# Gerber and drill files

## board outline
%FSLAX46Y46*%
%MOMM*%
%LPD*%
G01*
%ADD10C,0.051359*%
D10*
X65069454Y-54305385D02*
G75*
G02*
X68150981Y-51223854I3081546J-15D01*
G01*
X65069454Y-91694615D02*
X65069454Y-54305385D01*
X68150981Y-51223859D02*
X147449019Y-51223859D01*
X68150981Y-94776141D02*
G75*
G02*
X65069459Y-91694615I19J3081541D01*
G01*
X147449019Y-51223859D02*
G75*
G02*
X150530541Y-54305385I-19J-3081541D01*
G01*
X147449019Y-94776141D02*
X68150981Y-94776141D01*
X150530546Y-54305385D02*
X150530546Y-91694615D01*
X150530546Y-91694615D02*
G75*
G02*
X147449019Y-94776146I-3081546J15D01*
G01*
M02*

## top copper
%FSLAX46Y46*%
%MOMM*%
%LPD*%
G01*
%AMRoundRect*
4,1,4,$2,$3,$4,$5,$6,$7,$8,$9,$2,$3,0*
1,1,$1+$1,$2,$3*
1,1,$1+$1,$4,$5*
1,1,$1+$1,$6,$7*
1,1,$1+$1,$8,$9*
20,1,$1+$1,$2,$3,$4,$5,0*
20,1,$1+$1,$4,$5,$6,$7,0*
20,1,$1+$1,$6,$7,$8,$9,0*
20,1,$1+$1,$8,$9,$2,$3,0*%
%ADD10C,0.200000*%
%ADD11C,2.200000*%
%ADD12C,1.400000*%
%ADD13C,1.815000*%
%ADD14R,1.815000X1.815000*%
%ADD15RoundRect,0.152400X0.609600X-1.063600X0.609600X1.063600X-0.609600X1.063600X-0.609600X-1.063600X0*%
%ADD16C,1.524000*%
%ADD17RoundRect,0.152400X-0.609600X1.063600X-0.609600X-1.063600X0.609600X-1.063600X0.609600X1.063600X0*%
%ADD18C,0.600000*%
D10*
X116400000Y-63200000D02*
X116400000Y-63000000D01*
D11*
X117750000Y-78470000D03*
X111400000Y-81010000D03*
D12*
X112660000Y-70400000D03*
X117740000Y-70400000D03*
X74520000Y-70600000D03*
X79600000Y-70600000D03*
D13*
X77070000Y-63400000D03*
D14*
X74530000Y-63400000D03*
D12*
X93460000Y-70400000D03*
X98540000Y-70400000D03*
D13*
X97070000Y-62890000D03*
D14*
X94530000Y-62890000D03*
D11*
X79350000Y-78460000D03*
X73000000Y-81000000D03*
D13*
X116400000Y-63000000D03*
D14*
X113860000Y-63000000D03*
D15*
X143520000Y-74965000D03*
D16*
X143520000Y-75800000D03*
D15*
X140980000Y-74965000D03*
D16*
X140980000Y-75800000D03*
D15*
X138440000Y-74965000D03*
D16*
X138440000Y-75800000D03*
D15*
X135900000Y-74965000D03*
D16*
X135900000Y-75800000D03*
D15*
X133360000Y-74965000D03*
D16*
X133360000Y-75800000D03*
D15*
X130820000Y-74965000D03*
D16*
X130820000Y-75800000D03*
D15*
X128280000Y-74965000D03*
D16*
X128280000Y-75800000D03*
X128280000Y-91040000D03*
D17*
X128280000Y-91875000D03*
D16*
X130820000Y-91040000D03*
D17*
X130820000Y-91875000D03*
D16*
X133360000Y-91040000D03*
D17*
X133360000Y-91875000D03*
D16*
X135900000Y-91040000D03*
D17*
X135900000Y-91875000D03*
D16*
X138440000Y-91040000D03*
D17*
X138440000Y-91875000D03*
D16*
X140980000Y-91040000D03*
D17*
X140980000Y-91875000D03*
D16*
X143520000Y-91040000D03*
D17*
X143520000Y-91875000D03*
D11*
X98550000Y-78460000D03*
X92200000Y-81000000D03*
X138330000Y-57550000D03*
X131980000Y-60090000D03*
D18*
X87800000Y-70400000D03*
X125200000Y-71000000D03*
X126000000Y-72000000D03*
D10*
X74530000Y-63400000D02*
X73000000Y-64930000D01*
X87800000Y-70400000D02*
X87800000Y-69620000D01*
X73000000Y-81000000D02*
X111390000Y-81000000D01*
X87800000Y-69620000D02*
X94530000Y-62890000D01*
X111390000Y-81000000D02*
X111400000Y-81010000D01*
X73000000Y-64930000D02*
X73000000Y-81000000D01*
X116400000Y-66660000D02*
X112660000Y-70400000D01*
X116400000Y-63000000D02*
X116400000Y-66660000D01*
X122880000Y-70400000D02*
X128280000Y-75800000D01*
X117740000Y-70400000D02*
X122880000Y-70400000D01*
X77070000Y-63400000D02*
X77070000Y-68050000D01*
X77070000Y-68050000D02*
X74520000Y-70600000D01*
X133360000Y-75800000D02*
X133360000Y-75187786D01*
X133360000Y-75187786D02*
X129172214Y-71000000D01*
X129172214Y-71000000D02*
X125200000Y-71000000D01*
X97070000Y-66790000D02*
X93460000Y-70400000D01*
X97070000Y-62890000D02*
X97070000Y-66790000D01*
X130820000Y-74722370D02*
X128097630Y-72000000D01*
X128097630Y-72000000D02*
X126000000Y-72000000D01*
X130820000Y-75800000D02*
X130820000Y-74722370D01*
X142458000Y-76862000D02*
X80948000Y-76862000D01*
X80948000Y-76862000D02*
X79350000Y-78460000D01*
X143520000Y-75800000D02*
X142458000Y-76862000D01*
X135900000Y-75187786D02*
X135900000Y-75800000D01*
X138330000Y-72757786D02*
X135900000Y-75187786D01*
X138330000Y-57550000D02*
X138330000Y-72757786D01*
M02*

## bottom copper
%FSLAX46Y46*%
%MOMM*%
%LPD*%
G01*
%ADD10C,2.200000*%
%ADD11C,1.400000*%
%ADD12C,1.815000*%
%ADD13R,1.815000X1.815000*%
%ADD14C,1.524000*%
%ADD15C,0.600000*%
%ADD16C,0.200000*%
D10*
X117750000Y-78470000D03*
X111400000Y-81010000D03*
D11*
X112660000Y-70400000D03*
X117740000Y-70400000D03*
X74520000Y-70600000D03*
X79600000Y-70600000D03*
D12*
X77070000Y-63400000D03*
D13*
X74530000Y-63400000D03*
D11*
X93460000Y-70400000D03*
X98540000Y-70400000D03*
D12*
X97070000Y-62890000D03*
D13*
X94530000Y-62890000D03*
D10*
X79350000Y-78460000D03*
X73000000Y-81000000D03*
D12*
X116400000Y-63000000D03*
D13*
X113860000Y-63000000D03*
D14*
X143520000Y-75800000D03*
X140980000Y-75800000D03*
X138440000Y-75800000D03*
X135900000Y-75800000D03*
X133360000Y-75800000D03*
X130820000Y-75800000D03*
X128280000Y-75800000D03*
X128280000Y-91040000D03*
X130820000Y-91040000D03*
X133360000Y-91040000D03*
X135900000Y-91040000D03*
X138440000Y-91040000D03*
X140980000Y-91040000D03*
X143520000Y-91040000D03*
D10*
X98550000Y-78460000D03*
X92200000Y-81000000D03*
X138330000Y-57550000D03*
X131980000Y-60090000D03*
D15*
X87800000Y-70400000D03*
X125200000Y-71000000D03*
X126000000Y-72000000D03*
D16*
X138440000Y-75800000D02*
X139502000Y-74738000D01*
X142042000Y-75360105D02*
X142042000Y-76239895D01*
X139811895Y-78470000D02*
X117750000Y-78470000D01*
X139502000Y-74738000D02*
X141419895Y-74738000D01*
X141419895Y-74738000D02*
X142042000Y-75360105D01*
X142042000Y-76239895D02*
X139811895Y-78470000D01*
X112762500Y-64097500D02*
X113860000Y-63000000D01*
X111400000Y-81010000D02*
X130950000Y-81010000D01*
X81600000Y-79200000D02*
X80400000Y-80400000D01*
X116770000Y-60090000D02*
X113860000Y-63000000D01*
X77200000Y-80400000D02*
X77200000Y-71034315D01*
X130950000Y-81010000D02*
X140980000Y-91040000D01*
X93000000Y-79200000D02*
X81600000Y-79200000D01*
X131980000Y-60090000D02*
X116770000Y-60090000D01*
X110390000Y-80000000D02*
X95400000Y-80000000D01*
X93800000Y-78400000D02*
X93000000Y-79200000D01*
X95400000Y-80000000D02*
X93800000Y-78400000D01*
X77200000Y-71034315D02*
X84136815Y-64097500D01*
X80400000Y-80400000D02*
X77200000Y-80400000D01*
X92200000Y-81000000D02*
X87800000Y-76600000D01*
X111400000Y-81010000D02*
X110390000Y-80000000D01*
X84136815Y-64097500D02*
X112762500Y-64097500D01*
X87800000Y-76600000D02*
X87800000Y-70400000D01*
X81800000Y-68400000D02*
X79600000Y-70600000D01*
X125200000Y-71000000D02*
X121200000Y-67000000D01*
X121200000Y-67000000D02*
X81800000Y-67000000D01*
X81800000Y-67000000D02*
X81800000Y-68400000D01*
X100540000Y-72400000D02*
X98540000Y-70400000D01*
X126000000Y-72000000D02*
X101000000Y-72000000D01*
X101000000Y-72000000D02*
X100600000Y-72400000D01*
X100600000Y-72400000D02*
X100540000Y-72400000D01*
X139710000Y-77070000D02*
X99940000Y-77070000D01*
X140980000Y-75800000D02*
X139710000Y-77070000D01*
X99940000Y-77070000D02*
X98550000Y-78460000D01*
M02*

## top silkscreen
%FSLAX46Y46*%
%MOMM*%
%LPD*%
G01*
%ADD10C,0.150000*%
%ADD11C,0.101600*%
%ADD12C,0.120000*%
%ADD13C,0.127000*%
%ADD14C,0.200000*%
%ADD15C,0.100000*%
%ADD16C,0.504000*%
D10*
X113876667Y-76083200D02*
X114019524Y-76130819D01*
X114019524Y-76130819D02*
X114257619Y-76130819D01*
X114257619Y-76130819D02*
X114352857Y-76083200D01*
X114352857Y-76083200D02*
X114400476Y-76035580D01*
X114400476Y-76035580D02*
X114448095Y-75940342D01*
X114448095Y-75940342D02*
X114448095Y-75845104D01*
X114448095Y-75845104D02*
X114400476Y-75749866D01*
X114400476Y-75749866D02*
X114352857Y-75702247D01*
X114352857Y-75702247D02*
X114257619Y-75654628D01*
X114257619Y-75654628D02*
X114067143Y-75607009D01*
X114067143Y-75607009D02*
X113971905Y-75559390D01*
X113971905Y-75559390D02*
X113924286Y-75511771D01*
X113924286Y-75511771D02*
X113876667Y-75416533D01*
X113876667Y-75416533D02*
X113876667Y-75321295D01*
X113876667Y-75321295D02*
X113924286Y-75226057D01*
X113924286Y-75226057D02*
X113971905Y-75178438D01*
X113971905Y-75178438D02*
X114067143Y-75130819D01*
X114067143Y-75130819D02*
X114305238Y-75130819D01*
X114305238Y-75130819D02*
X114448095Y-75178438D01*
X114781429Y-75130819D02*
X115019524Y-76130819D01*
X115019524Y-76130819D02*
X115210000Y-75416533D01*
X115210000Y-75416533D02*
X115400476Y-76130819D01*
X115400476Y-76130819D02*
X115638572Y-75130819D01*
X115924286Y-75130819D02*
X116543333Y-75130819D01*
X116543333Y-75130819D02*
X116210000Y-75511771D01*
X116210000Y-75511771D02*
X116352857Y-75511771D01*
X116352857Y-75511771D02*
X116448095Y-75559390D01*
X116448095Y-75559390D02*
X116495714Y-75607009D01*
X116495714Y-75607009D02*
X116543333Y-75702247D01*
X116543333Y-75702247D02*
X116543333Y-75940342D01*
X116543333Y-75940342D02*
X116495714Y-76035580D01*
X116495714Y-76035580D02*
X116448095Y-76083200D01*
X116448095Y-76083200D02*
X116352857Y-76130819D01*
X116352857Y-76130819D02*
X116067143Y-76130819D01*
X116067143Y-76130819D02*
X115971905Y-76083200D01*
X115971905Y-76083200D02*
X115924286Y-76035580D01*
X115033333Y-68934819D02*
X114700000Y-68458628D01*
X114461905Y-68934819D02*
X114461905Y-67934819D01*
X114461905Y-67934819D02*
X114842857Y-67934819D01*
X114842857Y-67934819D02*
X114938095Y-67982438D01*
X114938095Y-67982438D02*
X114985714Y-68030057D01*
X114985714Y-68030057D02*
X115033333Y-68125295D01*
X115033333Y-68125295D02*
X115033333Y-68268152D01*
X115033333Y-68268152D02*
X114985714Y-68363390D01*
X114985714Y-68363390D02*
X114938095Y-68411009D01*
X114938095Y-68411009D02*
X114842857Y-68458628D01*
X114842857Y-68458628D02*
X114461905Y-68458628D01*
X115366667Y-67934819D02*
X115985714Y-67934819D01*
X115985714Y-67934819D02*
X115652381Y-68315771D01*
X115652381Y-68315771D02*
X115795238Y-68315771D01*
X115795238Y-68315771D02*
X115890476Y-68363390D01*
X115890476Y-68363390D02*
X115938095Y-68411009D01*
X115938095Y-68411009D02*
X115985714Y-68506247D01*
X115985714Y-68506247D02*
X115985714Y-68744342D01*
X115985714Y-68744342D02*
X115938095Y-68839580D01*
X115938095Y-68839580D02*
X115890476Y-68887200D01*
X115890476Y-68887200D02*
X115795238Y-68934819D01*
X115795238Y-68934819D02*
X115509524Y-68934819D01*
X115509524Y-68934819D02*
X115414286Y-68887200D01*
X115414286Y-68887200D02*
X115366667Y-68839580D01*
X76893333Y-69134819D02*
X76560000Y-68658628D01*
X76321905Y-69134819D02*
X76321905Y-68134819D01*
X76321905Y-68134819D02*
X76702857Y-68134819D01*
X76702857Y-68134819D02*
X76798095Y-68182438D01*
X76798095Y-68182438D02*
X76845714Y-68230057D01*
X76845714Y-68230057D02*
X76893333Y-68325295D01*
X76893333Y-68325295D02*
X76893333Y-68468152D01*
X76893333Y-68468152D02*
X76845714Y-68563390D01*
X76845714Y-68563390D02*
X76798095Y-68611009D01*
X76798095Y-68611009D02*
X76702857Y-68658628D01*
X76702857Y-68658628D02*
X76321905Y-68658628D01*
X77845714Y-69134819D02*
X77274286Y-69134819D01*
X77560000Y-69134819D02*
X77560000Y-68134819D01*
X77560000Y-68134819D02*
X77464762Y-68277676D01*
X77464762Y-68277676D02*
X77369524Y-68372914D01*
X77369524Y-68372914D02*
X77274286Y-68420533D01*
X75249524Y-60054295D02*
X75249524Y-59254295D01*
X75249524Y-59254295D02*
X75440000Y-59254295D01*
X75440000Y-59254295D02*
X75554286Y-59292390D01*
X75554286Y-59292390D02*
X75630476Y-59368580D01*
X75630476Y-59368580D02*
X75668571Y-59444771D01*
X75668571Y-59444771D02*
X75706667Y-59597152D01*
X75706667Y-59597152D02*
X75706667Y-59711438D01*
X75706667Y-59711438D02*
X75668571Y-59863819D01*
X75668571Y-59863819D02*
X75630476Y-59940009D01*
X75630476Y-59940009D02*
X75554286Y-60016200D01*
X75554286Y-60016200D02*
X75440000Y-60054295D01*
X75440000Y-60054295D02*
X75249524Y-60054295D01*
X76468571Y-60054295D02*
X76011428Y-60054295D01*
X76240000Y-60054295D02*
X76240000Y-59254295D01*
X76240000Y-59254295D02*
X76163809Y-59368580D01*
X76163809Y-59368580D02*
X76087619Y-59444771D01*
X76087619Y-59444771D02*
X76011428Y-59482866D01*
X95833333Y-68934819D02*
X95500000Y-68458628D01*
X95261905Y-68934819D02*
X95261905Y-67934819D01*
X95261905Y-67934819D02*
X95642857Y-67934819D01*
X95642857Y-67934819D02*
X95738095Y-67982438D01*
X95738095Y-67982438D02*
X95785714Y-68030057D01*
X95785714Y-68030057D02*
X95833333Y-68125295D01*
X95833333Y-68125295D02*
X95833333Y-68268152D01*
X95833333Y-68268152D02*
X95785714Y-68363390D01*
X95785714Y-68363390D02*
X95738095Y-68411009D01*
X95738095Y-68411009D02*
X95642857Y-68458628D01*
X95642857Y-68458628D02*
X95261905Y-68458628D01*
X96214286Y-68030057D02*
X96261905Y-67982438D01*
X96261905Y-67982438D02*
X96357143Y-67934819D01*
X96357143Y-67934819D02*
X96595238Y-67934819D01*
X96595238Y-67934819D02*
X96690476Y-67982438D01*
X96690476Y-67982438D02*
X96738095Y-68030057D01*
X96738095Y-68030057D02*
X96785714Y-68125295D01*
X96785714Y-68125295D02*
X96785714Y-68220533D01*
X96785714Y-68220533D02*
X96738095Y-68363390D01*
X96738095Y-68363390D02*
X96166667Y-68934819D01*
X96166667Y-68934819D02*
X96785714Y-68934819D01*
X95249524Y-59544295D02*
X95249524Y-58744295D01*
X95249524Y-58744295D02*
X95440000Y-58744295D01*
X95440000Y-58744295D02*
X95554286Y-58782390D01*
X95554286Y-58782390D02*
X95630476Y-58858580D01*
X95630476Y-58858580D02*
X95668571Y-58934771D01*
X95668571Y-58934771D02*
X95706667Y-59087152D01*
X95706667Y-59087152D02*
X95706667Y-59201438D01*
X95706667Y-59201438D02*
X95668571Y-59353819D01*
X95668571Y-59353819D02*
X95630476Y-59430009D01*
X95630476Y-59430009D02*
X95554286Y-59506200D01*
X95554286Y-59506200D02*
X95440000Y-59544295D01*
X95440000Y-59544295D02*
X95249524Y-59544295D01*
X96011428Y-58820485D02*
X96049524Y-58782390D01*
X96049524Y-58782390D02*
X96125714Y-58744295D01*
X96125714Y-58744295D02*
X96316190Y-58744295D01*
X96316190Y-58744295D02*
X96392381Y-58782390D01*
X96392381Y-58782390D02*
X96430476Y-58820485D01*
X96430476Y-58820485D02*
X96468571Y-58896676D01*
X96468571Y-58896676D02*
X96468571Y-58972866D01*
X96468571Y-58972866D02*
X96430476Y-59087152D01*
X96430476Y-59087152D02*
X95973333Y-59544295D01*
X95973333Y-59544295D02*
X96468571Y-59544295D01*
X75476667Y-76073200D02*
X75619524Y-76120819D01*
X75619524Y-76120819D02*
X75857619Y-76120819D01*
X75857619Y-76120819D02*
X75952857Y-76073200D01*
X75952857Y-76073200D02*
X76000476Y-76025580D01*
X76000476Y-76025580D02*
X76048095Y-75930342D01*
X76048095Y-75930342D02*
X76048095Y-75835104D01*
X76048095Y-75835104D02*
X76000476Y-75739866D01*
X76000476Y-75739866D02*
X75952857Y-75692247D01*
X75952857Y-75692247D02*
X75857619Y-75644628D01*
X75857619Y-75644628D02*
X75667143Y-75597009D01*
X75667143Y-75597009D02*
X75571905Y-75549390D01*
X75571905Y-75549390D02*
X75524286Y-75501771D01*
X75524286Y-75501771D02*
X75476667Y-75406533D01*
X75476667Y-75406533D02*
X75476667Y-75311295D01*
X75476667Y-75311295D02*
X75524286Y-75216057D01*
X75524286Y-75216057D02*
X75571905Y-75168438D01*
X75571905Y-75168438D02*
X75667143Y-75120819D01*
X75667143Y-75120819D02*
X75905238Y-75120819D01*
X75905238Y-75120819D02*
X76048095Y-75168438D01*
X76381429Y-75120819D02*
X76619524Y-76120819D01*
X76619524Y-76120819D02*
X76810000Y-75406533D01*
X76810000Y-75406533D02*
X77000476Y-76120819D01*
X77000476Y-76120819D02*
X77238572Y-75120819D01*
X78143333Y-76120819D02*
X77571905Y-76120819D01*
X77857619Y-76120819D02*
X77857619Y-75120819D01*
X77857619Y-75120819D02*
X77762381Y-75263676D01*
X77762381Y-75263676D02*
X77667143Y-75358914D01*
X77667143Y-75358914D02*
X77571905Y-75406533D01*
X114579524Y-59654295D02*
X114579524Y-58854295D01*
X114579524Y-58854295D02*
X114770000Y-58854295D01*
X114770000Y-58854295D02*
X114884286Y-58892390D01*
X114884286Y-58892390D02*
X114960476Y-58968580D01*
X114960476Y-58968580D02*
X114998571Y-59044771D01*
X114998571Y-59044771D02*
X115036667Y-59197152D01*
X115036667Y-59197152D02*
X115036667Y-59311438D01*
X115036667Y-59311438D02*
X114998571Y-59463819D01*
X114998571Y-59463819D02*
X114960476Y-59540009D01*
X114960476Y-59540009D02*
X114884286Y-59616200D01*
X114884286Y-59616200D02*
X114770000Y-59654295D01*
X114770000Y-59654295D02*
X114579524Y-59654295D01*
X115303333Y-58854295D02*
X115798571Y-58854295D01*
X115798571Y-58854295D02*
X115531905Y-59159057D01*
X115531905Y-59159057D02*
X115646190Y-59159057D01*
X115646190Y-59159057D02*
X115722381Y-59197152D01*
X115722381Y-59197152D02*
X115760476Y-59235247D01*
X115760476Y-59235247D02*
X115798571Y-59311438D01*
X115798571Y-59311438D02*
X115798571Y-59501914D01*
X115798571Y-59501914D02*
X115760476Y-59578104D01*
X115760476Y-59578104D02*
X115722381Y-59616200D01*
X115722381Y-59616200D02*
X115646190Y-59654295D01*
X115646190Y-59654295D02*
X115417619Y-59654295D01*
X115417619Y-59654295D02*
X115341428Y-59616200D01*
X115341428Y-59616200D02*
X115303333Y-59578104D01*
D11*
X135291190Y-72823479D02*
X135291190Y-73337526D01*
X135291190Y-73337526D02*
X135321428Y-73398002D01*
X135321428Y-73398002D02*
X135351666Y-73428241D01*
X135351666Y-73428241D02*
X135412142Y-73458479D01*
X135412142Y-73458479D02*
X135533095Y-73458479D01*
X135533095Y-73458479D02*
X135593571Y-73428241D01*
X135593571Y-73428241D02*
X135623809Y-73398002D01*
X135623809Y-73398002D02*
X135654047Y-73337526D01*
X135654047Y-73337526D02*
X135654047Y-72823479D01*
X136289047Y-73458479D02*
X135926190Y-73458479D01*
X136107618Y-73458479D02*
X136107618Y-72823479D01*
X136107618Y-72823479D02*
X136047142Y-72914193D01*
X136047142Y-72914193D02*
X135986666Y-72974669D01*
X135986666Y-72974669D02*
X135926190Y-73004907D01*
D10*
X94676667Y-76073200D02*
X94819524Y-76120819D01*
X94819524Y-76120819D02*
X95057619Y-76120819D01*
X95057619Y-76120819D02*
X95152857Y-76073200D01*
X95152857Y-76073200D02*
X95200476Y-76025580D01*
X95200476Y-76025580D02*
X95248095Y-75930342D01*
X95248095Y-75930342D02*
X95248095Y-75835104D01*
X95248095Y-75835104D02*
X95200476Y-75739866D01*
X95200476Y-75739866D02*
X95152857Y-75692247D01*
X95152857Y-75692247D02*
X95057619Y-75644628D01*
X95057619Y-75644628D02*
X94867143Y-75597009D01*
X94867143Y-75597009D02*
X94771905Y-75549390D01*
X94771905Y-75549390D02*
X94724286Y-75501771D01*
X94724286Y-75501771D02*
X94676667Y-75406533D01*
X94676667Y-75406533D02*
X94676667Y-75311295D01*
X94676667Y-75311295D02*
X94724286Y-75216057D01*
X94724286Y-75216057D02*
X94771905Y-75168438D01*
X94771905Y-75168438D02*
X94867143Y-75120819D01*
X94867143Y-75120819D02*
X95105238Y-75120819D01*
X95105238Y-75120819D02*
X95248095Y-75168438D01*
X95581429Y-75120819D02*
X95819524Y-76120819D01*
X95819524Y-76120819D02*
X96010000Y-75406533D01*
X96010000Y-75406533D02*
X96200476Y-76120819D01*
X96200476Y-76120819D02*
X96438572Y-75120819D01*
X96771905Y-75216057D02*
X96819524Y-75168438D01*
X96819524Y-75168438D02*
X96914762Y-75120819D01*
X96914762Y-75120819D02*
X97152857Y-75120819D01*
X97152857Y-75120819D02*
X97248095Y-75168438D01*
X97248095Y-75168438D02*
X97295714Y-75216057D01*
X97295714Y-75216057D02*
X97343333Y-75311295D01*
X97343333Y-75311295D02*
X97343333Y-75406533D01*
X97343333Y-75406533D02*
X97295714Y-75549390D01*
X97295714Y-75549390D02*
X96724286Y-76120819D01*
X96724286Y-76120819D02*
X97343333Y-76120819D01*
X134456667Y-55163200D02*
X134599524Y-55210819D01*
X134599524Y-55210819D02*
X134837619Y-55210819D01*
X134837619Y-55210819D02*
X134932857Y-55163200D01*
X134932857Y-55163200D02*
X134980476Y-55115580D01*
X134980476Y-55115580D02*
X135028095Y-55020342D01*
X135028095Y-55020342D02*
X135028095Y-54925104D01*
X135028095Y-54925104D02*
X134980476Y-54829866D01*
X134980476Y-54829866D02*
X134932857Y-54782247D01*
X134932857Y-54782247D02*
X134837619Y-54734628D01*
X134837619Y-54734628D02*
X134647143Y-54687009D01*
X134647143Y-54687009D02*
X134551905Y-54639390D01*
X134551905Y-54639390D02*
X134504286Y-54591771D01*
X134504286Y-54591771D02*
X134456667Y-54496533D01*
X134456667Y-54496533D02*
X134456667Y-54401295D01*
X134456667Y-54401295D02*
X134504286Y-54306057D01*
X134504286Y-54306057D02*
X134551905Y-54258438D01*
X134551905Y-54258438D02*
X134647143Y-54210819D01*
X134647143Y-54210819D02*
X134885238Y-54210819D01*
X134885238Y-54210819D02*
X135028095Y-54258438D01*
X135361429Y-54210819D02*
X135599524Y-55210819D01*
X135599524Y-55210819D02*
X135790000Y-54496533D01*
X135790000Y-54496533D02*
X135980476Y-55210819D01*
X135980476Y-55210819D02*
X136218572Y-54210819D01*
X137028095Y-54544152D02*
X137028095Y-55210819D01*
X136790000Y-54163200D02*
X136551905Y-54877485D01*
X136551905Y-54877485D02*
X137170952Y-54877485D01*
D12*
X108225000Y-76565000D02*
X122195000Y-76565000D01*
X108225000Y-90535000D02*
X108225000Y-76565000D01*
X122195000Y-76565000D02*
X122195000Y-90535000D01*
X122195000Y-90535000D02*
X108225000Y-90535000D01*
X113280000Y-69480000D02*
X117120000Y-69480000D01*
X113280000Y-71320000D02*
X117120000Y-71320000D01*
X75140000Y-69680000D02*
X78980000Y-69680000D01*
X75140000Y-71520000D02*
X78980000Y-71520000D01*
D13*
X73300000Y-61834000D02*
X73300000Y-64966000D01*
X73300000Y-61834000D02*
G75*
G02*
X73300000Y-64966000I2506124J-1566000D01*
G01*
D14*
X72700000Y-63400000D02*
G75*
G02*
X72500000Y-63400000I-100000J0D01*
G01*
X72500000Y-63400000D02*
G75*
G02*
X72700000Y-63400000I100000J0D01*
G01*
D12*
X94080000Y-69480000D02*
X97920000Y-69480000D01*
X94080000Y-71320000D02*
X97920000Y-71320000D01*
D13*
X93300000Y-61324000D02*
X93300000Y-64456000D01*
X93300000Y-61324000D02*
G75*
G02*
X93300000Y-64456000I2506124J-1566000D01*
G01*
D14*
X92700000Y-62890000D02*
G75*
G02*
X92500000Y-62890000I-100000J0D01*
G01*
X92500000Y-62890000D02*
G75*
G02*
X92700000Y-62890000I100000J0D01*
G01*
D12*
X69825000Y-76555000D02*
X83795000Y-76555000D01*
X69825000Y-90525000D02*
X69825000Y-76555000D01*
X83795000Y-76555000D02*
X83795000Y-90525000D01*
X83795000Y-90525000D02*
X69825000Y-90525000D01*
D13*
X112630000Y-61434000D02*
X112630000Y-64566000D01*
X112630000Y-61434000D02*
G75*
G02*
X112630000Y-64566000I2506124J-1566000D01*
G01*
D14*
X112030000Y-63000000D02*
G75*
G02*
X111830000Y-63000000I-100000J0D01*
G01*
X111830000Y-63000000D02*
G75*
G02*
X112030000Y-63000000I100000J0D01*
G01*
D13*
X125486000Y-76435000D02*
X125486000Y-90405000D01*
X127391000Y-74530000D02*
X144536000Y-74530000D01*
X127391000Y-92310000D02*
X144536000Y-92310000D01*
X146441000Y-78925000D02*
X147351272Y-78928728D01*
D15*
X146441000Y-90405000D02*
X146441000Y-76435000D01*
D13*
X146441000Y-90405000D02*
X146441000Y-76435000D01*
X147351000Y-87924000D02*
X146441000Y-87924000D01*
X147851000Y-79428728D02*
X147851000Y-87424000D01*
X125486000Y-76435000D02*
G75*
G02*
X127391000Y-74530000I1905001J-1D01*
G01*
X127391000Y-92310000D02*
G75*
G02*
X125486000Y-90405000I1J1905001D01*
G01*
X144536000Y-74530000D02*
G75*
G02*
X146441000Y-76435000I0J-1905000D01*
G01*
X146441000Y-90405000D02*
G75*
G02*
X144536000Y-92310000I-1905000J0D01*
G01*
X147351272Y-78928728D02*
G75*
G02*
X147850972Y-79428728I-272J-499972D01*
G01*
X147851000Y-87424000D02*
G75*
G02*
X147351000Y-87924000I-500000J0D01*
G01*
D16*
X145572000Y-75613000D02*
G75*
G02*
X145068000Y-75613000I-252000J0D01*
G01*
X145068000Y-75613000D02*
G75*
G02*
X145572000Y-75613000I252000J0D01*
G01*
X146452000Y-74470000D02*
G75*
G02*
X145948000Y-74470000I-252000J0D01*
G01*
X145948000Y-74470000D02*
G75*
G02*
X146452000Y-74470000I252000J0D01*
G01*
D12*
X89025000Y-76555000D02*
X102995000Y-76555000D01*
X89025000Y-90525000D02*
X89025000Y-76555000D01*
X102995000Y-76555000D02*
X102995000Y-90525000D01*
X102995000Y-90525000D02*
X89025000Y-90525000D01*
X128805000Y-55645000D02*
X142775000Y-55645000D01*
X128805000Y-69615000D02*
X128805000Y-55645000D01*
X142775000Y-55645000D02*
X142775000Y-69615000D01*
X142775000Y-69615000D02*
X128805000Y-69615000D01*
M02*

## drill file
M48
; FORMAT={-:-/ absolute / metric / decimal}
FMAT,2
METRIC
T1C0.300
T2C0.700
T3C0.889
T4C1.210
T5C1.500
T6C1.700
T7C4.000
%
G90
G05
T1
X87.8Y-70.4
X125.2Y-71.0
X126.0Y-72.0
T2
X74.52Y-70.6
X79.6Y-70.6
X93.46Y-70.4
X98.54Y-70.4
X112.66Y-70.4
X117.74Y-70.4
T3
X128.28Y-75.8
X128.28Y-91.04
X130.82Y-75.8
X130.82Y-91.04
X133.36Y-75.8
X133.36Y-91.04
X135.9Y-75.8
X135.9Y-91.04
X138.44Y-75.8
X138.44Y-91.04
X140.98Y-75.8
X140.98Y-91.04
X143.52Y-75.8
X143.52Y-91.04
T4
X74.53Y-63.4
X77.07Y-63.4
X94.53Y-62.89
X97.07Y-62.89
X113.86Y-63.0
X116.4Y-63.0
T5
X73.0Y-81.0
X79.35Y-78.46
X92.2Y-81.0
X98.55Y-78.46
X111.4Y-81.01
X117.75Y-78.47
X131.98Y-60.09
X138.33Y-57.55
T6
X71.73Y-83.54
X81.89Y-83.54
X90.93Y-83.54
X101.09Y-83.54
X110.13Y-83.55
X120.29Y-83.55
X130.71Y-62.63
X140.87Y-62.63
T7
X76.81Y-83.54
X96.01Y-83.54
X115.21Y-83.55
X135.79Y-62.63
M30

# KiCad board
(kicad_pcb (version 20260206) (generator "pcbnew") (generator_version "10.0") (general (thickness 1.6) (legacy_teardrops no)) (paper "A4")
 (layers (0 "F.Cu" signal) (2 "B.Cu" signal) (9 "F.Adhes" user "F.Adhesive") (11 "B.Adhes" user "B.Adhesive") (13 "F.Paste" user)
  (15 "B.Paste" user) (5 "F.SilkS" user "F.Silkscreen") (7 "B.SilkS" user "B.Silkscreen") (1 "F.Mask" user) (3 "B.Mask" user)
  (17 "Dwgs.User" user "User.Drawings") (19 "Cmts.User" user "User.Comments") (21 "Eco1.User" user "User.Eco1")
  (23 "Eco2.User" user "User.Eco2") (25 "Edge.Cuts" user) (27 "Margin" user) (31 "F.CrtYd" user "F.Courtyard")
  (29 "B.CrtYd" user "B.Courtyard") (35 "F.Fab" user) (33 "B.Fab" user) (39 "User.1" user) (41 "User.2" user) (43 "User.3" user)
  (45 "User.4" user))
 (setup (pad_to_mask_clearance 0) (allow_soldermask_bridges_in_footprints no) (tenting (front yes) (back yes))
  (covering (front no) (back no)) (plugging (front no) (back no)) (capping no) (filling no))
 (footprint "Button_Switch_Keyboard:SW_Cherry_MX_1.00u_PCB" (layer "F.Cu") (at 117.75 78.47)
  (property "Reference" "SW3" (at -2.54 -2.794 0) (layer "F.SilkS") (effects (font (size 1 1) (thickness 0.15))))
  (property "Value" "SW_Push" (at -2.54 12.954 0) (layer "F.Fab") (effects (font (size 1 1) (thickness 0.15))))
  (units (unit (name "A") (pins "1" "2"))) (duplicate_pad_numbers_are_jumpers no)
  (fp_line (start -9.525 -1.905) (end 4.445 -1.905) (stroke (width 0.12) (type solid)) (layer "F.SilkS"))
  (fp_line (start -9.525 12.065) (end -9.525 -1.905) (stroke (width 0.12) (type solid)) (layer "F.SilkS"))
  (fp_line (start 4.445 -1.905) (end 4.445 12.065) (stroke (width 0.12) (type solid)) (layer "F.SilkS"))
  (fp_line (start 4.445 12.065) (end -9.525 12.065) (stroke (width 0.12) (type solid)) (layer "F.SilkS"))
  (pad "" np_thru_hole circle (at -7.62 5.08) (size 1.7 1.7) (drill 1.7) (layers "*.Cu" "*.Mask"))
  (pad "" np_thru_hole circle (at -2.54 5.08) (size 4 4) (drill 4) (layers "*.Cu" "*.Mask"))
  (pad "" np_thru_hole circle (at 2.54 5.08) (size 1.7 1.7) (drill 1.7) (layers "*.Cu" "*.Mask"))
  (pad "1" thru_hole circle (at 0 0) (size 2.2 2.2) (drill 1.5) (layers "*.Cu" "*.Mask") (remove_unused_layers no)
   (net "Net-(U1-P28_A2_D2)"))
  (pad "2" thru_hole circle (at -6.35 2.54) (size 2.2 2.2) (drill 1.5) (layers "*.Cu" "*.Mask") (remove_unused_layers no) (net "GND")))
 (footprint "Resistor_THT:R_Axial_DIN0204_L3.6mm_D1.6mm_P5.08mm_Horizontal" (layer "F.Cu") (at 112.66 70.4)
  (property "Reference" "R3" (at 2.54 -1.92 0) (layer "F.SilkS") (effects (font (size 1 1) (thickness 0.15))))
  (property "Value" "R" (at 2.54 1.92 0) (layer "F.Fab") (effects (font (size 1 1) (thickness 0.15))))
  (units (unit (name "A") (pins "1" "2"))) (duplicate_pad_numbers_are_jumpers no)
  (fp_line (start 0.62 -0.92) (end 4.46 -0.92) (stroke (width 0.12) (type solid)) (layer "F.SilkS"))
  (fp_line (start 0.62 0.92) (end 4.46 0.92) (stroke (width 0.12) (type solid)) (layer "F.SilkS"))
  (pad "1" thru_hole circle (at 0 0) (size 1.4 1.4) (drill 0.7) (layers "*.Cu" "*.Mask") (remove_unused_layers no) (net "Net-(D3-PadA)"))
  (pad "2" thru_hole circle (at 5.08 0) (size 1.4 1.4) (drill 0.7) (layers "*.Cu" "*.Mask") (remove_unused_layers no)
   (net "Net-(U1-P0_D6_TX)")))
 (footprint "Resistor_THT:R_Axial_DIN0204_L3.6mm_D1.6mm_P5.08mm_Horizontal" (layer "F.Cu") (at 74.52 70.6)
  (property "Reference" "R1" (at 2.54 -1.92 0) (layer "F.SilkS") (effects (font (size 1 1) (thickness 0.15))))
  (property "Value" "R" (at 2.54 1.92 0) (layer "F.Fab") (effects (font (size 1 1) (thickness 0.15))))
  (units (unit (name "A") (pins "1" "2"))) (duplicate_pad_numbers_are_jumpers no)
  (fp_line (start 0.62 -0.92) (end 4.46 -0.92) (stroke (width 0.12) (type solid)) (layer "F.SilkS"))
  (fp_line (start 0.62 0.92) (end 4.46 0.92) (stroke (width 0.12) (type solid)) (layer "F.SilkS"))
  (pad "1" thru_hole circle (at 0 0) (size 1.4 1.4) (drill 0.7) (layers "*.Cu" "*.Mask") (remove_unused_layers no) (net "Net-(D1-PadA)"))
  (pad "2" thru_hole circle (at 5.08 0) (size 1.4 1.4) (drill 0.7) (layers "*.Cu" "*.Mask") (remove_unused_layers no)
   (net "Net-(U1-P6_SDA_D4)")))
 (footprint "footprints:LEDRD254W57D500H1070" (layer "F.Cu") (at 75.8 63.4)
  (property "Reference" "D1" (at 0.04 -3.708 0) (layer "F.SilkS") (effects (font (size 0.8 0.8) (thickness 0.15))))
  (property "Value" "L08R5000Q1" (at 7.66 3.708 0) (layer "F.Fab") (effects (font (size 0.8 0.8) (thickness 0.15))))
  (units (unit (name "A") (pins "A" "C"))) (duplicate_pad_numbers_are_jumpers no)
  (fp_line (start -2.5 -1.566) (end -2.5 1.566) (stroke (width 0.127) (type solid)) (layer "F.SilkS"))
  (fp_arc (start -2.5 -1.566) (mid 2.961291 0) (end -2.5 1.566) (stroke (width 0.127) (type solid)) (layer "F.SilkS"))
  (fp_circle (center -3.2 0) (end -3.1 0) (stroke (width 0.2) (type solid)) (fill no) (layer "F.SilkS"))
  (pad "A" thru_hole circle (at 1.27 0) (size 1.815 1.815) (drill 1.21) (layers "*.Cu" "*.Mask") (remove_unused_layers no)
   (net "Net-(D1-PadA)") (solder_mask_margin 0.102))
  (pad "C" thru_hole rect (at -1.27 0) (size 1.815 1.815) (drill 1.21) (layers "*.Cu" "*.Mask") (remove_unused_layers no) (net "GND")
   (solder_mask_margin 0.102)))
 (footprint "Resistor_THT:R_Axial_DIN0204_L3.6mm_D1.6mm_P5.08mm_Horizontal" (layer "F.Cu") (at 93.46 70.4)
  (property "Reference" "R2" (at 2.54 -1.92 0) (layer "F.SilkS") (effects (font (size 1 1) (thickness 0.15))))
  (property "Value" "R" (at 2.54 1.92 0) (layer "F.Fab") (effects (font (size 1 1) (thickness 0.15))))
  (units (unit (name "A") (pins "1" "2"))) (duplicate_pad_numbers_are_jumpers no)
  (fp_line (start 0.62 -0.92) (end 4.46 -0.92) (stroke (width 0.12) (type solid)) (layer "F.SilkS"))
  (fp_line (start 0.62 0.92) (end 4.46 0.92) (stroke (width 0.12) (type solid)) (layer "F.SilkS"))
  (pad "1" thru_hole circle (at 0 0) (size 1.4 1.4) (drill 0.7) (layers "*.Cu" "*.Mask") (remove_unused_layers no) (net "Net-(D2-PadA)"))
  (pad "2" thru_hole circle (at 5.08 0) (size 1.4 1.4) (drill 0.7) (layers "*.Cu" "*.Mask") (remove_unused_layers no)
   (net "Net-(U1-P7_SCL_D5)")))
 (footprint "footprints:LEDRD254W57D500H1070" (layer "F.Cu") (at 95.8 62.89)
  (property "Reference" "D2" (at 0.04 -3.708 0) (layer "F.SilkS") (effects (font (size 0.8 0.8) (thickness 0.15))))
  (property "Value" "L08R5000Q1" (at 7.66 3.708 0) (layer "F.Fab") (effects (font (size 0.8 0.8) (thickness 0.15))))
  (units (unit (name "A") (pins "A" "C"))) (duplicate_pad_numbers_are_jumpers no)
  (fp_line (start -2.5 -1.566) (end -2.5 1.566) (stroke (width 0.127) (type solid)) (layer "F.SilkS"))
  (fp_arc (start -2.5 -1.566) (mid 2.961291 0) (end -2.5 1.566) (stroke (width 0.127) (type solid)) (layer "F.SilkS"))
  (fp_circle (center -3.2 0) (end -3.1 0) (stroke (width 0.2) (type solid)) (fill no) (layer "F.SilkS"))
  (pad "A" thru_hole circle (at 1.27 0) (size 1.815 1.815) (drill 1.21) (layers "*.Cu" "*.Mask") (remove_unused_layers no)
   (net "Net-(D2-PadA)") (solder_mask_margin 0.102))
  (pad "C" thru_hole rect (at -1.27 0) (size 1.815 1.815) (drill 1.21) (layers "*.Cu" "*.Mask") (remove_unused_layers no) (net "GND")
   (solder_mask_margin 0.102)))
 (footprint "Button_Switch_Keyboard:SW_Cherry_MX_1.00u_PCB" (layer "F.Cu") (at 79.35 78.46)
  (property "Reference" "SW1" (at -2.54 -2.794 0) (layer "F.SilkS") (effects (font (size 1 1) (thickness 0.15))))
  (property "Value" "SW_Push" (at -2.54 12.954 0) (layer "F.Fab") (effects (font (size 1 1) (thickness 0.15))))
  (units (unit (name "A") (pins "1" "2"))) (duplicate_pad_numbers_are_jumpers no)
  (fp_line (start -9.525 -1.905) (end 4.445 -1.905) (stroke (width 0.12) (type solid)) (layer "F.SilkS"))
  (fp_line (start -9.525 12.065) (end -9.525 -1.905) (stroke (width 0.12) (type solid)) (layer "F.SilkS"))
  (fp_line (start 4.445 -1.905) (end 4.445 12.065) (stroke (width 0.12) (type solid)) (layer "F.SilkS"))
  (fp_line (start 4.445 12.065) (end -9.525 12.065) (stroke (width 0.12) (type solid)) (layer "F.SilkS"))
  (pad "" np_thru_hole circle (at -7.62 5.08) (size 1.7 1.7) (drill 1.7) (layers "*.Cu" "*.Mask"))
  (pad "" np_thru_hole circle (at -2.54 5.08) (size 4 4) (drill 4) (layers "*.Cu" "*.Mask"))
  (pad "" np_thru_hole circle (at 2.54 5.08) (size 1.7 1.7) (drill 1.7) (layers "*.Cu" "*.Mask"))
  (pad "1" thru_hole circle (at 0 0) (size 2.2 2.2) (drill 1.5) (layers "*.Cu" "*.Mask") (remove_unused_layers no)
   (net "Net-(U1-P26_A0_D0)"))
  (pad "2" thru_hole circle (at -6.35 2.54) (size 2.2 2.2) (drill 1.5) (layers "*.Cu" "*.Mask") (remove_unused_layers no) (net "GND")))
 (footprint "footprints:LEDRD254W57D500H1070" (layer "F.Cu") (at 115.13 63)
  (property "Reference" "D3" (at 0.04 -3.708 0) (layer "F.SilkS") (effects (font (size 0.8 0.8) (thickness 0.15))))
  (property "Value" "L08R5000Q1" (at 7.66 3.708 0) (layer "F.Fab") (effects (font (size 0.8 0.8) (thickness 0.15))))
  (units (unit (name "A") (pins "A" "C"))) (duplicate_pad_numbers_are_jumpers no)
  (fp_line (start -2.5 -1.566) (end -2.5 1.566) (stroke (width 0.127) (type solid)) (layer "F.SilkS"))
  (fp_arc (start -2.5 -1.566) (mid 2.961291 0) (end -2.5 1.566) (stroke (width 0.127) (type solid)) (layer "F.SilkS"))
  (fp_circle (center -3.2 0) (end -3.1 0) (stroke (width 0.2) (type solid)) (fill no) (layer "F.SilkS"))
  (pad "A" thru_hole circle (at 1.27 0) (size 1.815 1.815) (drill 1.21) (layers "*.Cu" "*.Mask") (remove_unused_layers no)
   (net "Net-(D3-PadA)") (solder_mask_margin 0.102))
  (pad "C" thru_hole rect (at -1.27 0) (size 1.815 1.815) (drill 1.21) (layers "*.Cu" "*.Mask") (remove_unused_layers no) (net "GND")
   (solder_mask_margin 0.102)))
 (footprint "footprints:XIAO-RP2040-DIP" (layer "F.Cu") (at 135.9 83.42)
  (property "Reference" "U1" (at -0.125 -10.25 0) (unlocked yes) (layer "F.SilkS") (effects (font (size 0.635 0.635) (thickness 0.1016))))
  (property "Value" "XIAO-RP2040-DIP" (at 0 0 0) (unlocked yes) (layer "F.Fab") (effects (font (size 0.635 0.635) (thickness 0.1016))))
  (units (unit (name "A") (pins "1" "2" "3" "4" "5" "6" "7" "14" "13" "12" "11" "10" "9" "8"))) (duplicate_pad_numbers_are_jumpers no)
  (fp_line (start -10.414 -6.985) (end -10.414 6.985) (stroke (width 0.127) (type solid)) (layer "F.SilkS"))
  (fp_line (start -8.509 -8.89) (end 8.636 -8.89) (stroke (width 0.127) (type solid)) (layer "F.SilkS"))
  (fp_line (start -8.509 8.89) (end 8.636 8.89) (stroke (width 0.127) (type solid)) (layer "F.SilkS"))
  (fp_line (start 10.541 -4.495) (end 11.451272 -4.491272) (stroke (width 0.127) (type solid)) (layer "F.SilkS"))
  (fp_line (start 10.541 6.985) (end 10.541 -6.985) (stroke (width 0.1) (type solid)) (layer "F.SilkS"))
  (fp_line (start 10.541 6.985) (end 10.541 -6.985) (stroke (width 0.127) (type solid)) (layer "F.SilkS"))
  (fp_line (start 11.451 4.504) (end 10.541 4.504) (stroke (width 0.127) (type solid)) (layer "F.SilkS"))
  (fp_line (start 11.951 -3.991272) (end 11.951 4.004) (stroke (width 0.127) (type solid)) (layer "F.SilkS"))
  (fp_arc (start -10.414 -6.985) (mid -9.856038 -8.332038) (end -8.509 -8.89) (stroke (width 0.127) (type solid)) (layer "F.SilkS"))
  (fp_arc (start -8.509 8.89) (mid -9.856038 8.332038) (end -10.414 6.985) (stroke (width 0.127) (type solid)) (layer "F.SilkS"))
  (fp_arc (start 8.636 -8.89) (mid 9.983038 -8.332038) (end 10.541 -6.985) (stroke (width 0.127) (type solid)) (layer "F.SilkS"))
  (fp_arc (start 10.541 6.985) (mid 9.983038 8.332038) (end 8.636 8.89) (stroke (width 0.127) (type solid)) (layer "F.SilkS"))
  (fp_arc (start 11.451272 -4.491272) (mid 11.804644 -4.344724) (end 11.951 -3.991272) (stroke (width 0.127) (type default))
   (layer "F.SilkS"))
  (fp_arc (start 11.951 4.004) (mid 11.804553 4.357553) (end 11.451 4.504) (stroke (width 0.127) (type default)) (layer "F.SilkS"))
  (fp_circle (center 9.42 -7.807) (end 9.674 -7.807) (stroke (width 0.5) (type solid)) (fill yes) (layer "F.SilkS"))
  (fp_circle (center 10.3 -8.95) (end 10.554 -8.95) (stroke (width 0.5) (type solid)) (fill yes) (layer "F.SilkS"))
  (pad "1" smd roundrect (at 7.62 -8.455 90) (size 2.432 1.524) (layers "F.Cu" "F.Mask") (roundrect_rratio 0.1) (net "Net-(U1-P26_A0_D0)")
   (thermal_bridge_angle 45))
  (pad "1" thru_hole circle (at 7.62 -7.62 90) (size 1.524 1.524) (drill 0.889) (layers "*.Cu" "*.Mask") (remove_unused_layers no)
   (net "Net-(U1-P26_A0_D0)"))
  (pad "2" smd roundrect (at 5.08 -8.455 90) (size 2.432 1.524) (layers "F.Cu" "F.Mask") (roundrect_rratio 0.1) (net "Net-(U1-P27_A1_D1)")
   (thermal_bridge_angle 45))
  (pad "2" thru_hole circle (at 5.08 -7.62 90) (size 1.524 1.524) (drill 0.889) (layers "*.Cu" "*.Mask") (remove_unused_layers no)
   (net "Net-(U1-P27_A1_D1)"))
  (pad "3" smd roundrect (at 2.54 -8.455 90) (size 2.432 1.524) (layers "F.Cu" "F.Mask") (roundrect_rratio 0.1) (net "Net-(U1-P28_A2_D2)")
   (thermal_bridge_angle 45))
  (pad "3" thru_hole circle (at 2.54 -7.62 90) (size 1.524 1.524) (drill 0.889) (layers "*.Cu" "*.Mask") (remove_unused_layers no)
   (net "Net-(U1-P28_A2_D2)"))
  (pad "4" smd roundrect (at 0 -8.455 90) (size 2.432 1.524) (layers "F.Cu" "F.Mask") (roundrect_rratio 0.1) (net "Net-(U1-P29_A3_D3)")
   (thermal_bridge_angle 45))
  (pad "4" thru_hole circle (at 0 -7.62 90) (size 1.524 1.524) (drill 0.889) (layers "*.Cu" "*.Mask") (remove_unused_layers no)
   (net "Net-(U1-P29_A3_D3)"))
  (pad "5" smd roundrect (at -2.54 -8.455 90) (size 2.432 1.524) (layers "F.Cu" "F.Mask") (roundrect_rratio 0.1) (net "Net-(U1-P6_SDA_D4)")
   (thermal_bridge_angle 45))
  (pad "5" thru_hole circle (at -2.54 -7.62 90) (size 1.524 1.524) (drill 0.889) (layers "*.Cu" "*.Mask") (remove_unused_layers no)
   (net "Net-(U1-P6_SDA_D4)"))
  (pad "6" smd roundrect (at -5.08 -8.455 90) (size 2.432 1.524) (layers "F.Cu" "F.Mask") (roundrect_rratio 0.1) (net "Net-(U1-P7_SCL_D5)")
   (thermal_bridge_angle 45))
  (pad "6" thru_hole circle (at -5.08 -7.62 90) (size 1.524 1.524) (drill 0.889) (layers "*.Cu" "*.Mask") (remove_unused_layers no)
   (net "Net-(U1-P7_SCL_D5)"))
  (pad "7" smd roundrect (at -7.62 -8.455 90) (size 2.432 1.524) (layers "F.Cu" "F.Mask") (roundrect_rratio 0.1) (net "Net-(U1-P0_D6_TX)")
   (thermal_bridge_angle 45))
  (pad "7" thru_hole circle (at -7.62 -7.62 90) (size 1.524 1.524) (drill 0.889) (layers "*.Cu" "*.Mask") (remove_unused_layers no)
   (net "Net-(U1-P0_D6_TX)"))
  (pad "8" thru_hole circle (at -7.62 7.62 270) (size 1.524 1.524) (drill 0.889) (layers "*.Cu" "*.Mask") (remove_unused_layers no)
   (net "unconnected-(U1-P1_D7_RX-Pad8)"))
  (pad "8" smd roundrect (at -7.62 8.455 270) (size 2.432 1.524) (layers "F.Cu" "F.Mask") (roundrect_rratio 0.1)
   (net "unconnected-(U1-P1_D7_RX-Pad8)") (thermal_bridge_angle 45))
  (pad "9" thru_hole circle (at -5.08 7.62 270) (size 1.524 1.524) (drill 0.889) (layers "*.Cu" "*.Mask") (remove_unused_layers no)
   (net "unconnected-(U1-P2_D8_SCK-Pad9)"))
  (pad "9" smd roundrect (at -5.08 8.455 270) (size 2.432 1.524) (layers "F.Cu" "F.Mask") (roundrect_rratio 0.1)
   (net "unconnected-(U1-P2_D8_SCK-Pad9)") (thermal_bridge_angle 45))
  (pad "10" thru_hole circle (at -2.54 7.62 270) (size 1.524 1.524) (drill 0.889) (layers "*.Cu" "*.Mask") (remove_unused_layers no)
   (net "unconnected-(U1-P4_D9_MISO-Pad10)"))
  (pad "10" smd roundrect (at -2.54 8.455 270) (size 2.432 1.524) (layers "F.Cu" "F.Mask") (roundrect_rratio 0.1)
   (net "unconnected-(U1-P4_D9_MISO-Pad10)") (thermal_bridge_angle 45))
  (pad "11" thru_hole circle (at 0 7.62 270) (size 1.524 1.524) (drill 0.889) (layers "*.Cu" "*.Mask") (remove_unused_layers no)
   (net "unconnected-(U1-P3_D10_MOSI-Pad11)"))
  (pad "11" smd roundrect (at 0 8.455 270) (size 2.432 1.524) (layers "F.Cu" "F.Mask") (roundrect_rratio 0.1)
   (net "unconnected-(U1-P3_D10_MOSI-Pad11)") (thermal_bridge_angle 45))
  (pad "12" thru_hole circle (at 2.54 7.62 270) (size 1.524 1.524) (drill 0.889) (layers "*.Cu" "*.Mask") (remove_unused_layers no)
   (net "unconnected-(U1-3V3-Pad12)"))
  (pad "12" smd roundrect (at 2.54 8.455 270) (size 2.432 1.524) (layers "F.Cu" "F.Mask") (roundrect_rratio 0.1)
   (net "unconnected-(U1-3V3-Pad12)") (thermal_bridge_angle 45))
  (pad "13" thru_hole circle (at 5.08 7.62 270) (size 1.524 1.524) (drill 0.889) (layers "*.Cu" "*.Mask") (remove_unused_layers no)
   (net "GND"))
  (pad "13" smd roundrect (at 5.08 8.455 270) (size 2.432 1.524) (layers "F.Cu" "F.Mask") (roundrect_rratio 0.1) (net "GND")
   (thermal_bridge_angle 45))
  (pad "14" thru_hole circle (at 7.62 7.62 270) (size 1.524 1.524) (drill 0.889) (layers "*.Cu" "*.Mask") (remove_unused_layers no)
   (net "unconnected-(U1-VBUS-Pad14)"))
  (pad "14" smd roundrect (at 7.62 8.455 270) (size 2.432 1.524) (layers "F.Cu" "F.Mask") (roundrect_rratio 0.1)
   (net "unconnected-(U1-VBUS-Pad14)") (thermal_bridge_angle 45)))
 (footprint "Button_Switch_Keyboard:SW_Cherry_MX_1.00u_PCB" (layer "F.Cu") (at 98.55 78.46)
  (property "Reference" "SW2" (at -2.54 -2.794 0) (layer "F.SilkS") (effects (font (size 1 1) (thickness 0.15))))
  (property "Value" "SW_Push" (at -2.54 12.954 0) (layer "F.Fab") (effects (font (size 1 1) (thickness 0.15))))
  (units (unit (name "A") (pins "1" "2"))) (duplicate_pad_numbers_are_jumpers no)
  (fp_line (start -9.525 -1.905) (end 4.445 -1.905) (stroke (width 0.12) (type solid)) (layer "F.SilkS"))
  (fp_line (start -9.525 12.065) (end -9.525 -1.905) (stroke (width 0.12) (type solid)) (layer "F.SilkS"))
  (fp_line (start 4.445 -1.905) (end 4.445 12.065) (stroke (width 0.12) (type solid)) (layer "F.SilkS"))
  (fp_line (start 4.445 12.065) (end -9.525 12.065) (stroke (width 0.12) (type solid)) (layer "F.SilkS"))
  (pad "" np_thru_hole circle (at -7.62 5.08) (size 1.7 1.7) (drill 1.7) (layers "*.Cu" "*.Mask"))
  (pad "" np_thru_hole circle (at -2.54 5.08) (size 4 4) (drill 4) (layers "*.Cu" "*.Mask"))
  (pad "" np_thru_hole circle (at 2.54 5.08) (size 1.7 1.7) (drill 1.7) (layers "*.Cu" "*.Mask"))
  (pad "1" thru_hole circle (at 0 0) (size 2.2 2.2) (drill 1.5) (layers "*.Cu" "*.Mask") (remove_unused_layers no)
   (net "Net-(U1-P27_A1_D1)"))
  (pad "2" thru_hole circle (at -6.35 2.54) (size 2.2 2.2) (drill 1.5) (layers "*.Cu" "*.Mask") (remove_unused_layers no) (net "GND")))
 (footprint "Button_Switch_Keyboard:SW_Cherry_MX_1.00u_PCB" (layer "F.Cu") (at 138.33 57.55)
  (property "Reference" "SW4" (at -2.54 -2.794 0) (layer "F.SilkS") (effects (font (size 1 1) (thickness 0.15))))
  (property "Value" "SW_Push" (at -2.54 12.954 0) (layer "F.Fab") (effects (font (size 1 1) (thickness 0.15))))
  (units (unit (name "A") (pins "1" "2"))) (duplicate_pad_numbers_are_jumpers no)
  (fp_line (start -9.525 -1.905) (end 4.445 -1.905) (stroke (width 0.12) (type solid)) (layer "F.SilkS"))
  (fp_line (start -9.525 12.065) (end -9.525 -1.905) (stroke (width 0.12) (type solid)) (layer "F.SilkS"))
  (fp_line (start 4.445 -1.905) (end 4.445 12.065) (stroke (width 0.12) (type solid)) (layer "F.SilkS"))
  (fp_line (start 4.445 12.065) (end -9.525 12.065) (stroke (width 0.12) (type solid)) (layer "F.SilkS"))
  (pad "" np_thru_hole circle (at -7.62 5.08) (size 1.7 1.7) (drill 1.7) (layers "*.Cu" "*.Mask"))
  (pad "" np_thru_hole circle (at -2.54 5.08) (size 4 4) (drill 4) (layers "*.Cu" "*.Mask"))
  (pad "" np_thru_hole circle (at 2.54 5.08) (size 1.7 1.7) (drill 1.7) (layers "*.Cu" "*.Mask"))
  (pad "1" thru_hole circle (at 0 0) (size 2.2 2.2) (drill 1.5) (layers "*.Cu" "*.Mask") (remove_unused_layers no)
   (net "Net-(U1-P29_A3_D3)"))
  (pad "2" thru_hole circle (at -6.35 2.54) (size 2.2 2.2) (drill 1.5) (layers "*.Cu" "*.Mask") (remove_unused_layers no) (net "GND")))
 (gr_line (start 116.4 63.2) (end 116.4 63) (stroke (width 0.2) (type default)) (layer "F.Cu") (net "Net-(D3-PadA)"))
 (gr_arc (start 65.069454 54.305385) (mid 65.972012 52.126416) (end 68.150981 51.223859) (stroke (width 0.051359) (type default))
  (layer "Edge.Cuts"))
 (gr_line (start 65.069454 91.694615) (end 65.069454 54.305385) (stroke (width 0.051359) (type default)) (layer "Edge.Cuts"))
 (gr_line (start 68.150981 51.223859) (end 147.449019 51.223859) (stroke (width 0.051359) (type default)) (layer "Edge.Cuts"))
 (gr_arc (start 68.150981 94.776141) (mid 65.972013 93.873583) (end 65.069454 91.694615) (stroke (width 0.051359) (type default))
  (layer "Edge.Cuts"))
 (gr_arc (start 147.449019 51.223859) (mid 149.627987 52.126417) (end 150.530546 54.305385) (stroke (width 0.051359) (type default))
  (layer "Edge.Cuts"))
 (gr_line (start 147.449019 94.776141) (end 68.150981 94.776141) (stroke (width 0.051359) (type default)) (layer "Edge.Cuts"))
 (gr_line (start 150.530546 54.305385) (end 150.530546 91.694615) (stroke (width 0.051359) (type default)) (layer "Edge.Cuts"))
 (gr_arc (start 150.530546 91.694615) (mid 149.627988 93.873584) (end 147.449019 94.776141) (stroke (width 0.051359) (type default))
  (layer "Edge.Cuts"))
 (segment (start 138.44 75.8) (end 139.502 74.738) (width 0.2) (layer "B.Cu") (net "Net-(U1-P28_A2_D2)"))
 (segment (start 142.042 75.360105) (end 142.042 76.239895) (width 0.2) (layer "B.Cu") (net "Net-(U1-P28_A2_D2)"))
 (segment (start 139.811895 78.47) (end 117.75 78.47) (width 0.2) (layer "B.Cu") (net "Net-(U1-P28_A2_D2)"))
 (segment (start 139.502 74.738) (end 141.419895 74.738) (width 0.2) (layer "B.Cu") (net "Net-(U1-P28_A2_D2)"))
 (segment (start 141.419895 74.738) (end 142.042 75.360105) (width 0.2) (layer "B.Cu") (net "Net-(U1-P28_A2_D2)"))
 (segment (start 142.042 76.239895) (end 139.811895 78.47) (width 0.2) (layer "B.Cu") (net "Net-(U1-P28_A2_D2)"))
 (segment (start 74.53 63.4) (end 73 64.93) (width 0.2) (layer "F.Cu") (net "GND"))
 (segment (start 87.8 70.4) (end 87.8 69.62) (width 0.2) (layer "F.Cu") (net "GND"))
 (segment (start 73 81) (end 111.39 81) (width 0.2) (layer "F.Cu") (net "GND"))
 (segment (start 87.8 69.62) (end 94.53 62.89) (width 0.2) (layer "F.Cu") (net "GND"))
 (segment (start 111.39 81) (end 111.4 81.01) (width 0.2) (layer "F.Cu") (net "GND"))
 (segment (start 73 64.93) (end 73 81) (width 0.2) (layer "F.Cu") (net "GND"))
 (via (at 87.8 70.4) (size 0.6) (drill 0.3) (layers "F.Cu" "B.Cu") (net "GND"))
 (segment (start 112.7625 64.0975) (end 113.86 63) (width 0.2) (layer "B.Cu") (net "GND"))
 (segment (start 111.4 81.01) (end 130.95 81.01) (width 0.2) (layer "B.Cu") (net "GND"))
 (segment (start 81.6 79.2) (end 80.4 80.4) (width 0.2) (layer "B.Cu") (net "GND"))
 (segment (start 116.77 60.09) (end 113.86 63) (width 0.2) (layer "B.Cu") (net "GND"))
 (segment (start 77.2 80.4) (end 77.2 71.034315) (width 0.2) (layer "B.Cu") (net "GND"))
 (segment (start 130.95 81.01) (end 140.98 91.04) (width 0.2) (layer "B.Cu") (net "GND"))
 (segment (start 93 79.2) (end 81.6 79.2) (width 0.2) (layer "B.Cu") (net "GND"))
 (segment (start 131.98 60.09) (end 116.77 60.09) (width 0.2) (layer "B.Cu") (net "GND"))
 (segment (start 110.39 80) (end 95.4 80) (width 0.2) (layer "B.Cu") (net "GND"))
 (segment (start 93.8 78.4) (end 93 79.2) (width 0.2) (layer "B.Cu") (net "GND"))
 (segment (start 95.4 80) (end 93.8 78.4) (width 0.2) (layer "B.Cu") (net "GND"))
 (segment (start 77.2 71.034315) (end 84.136815 64.0975) (width 0.2) (layer "B.Cu") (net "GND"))
 (segment (start 80.4 80.4) (end 77.2 80.4) (width 0.2) (layer "B.Cu") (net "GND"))
 (segment (start 92.2 81) (end 87.8 76.6) (width 0.2) (layer "B.Cu") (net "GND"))
 (segment (start 111.4 81.01) (end 110.39 80) (width 0.2) (layer "B.Cu") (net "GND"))
 (segment (start 84.136815 64.0975) (end 112.7625 64.0975) (width 0.2) (layer "B.Cu") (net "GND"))
 (segment (start 87.8 76.6) (end 87.8 70.4) (width 0.2) (layer "B.Cu") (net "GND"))
 (segment (start 116.4 66.66) (end 112.66 70.4) (width 0.2) (layer "F.Cu") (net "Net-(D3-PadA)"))
 (segment (start 116.4 63) (end 116.4 66.66) (width 0.2) (layer "F.Cu") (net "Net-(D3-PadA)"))
 (segment (start 122.88 70.4) (end 128.28 75.8) (width 0.2) (layer "F.Cu") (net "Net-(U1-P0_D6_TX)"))
 (segment (start 117.74 70.4) (end 122.88 70.4) (width 0.2) (layer "F.Cu") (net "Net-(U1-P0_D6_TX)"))
 (segment (start 77.07 63.4) (end 77.07 68.05) (width 0.2) (layer "F.Cu") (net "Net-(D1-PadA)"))
 (segment (start 77.07 68.05) (end 74.52 70.6) (width 0.2) (layer "F.Cu") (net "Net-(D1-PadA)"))
 (segment (start 133.36 75.8) (end 133.36 75.187786) (width 0.2) (layer "F.Cu") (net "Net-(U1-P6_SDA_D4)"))
 (segment (start 133.36 75.187786) (end 129.172214 71) (width 0.2) (layer "F.Cu") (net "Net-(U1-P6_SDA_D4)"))
 (segment (start 129.172214 71) (end 125.2 71) (width 0.2) (layer "F.Cu") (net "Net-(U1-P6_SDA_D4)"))
 (via (at 125.2 71) (size 0.6) (drill 0.3) (layers "F.Cu" "B.Cu") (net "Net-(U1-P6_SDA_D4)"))
 (segment (start 81.8 68.4) (end 79.6 70.6) (width 0.2) (layer "B.Cu") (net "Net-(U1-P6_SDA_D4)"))
 (segment (start 125.2 71) (end 121.2 67) (width 0.2) (layer "B.Cu") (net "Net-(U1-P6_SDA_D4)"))
 (segment (start 121.2 67) (end 81.8 67) (width 0.2) (layer "B.Cu") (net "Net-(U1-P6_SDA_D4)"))
 (segment (start 81.8 67) (end 81.8 68.4) (width 0.2) (layer "B.Cu") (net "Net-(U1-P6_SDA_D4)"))
 (segment (start 97.07 66.79) (end 93.46 70.4) (width 0.2) (layer "F.Cu") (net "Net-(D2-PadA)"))
 (segment (start 97.07 62.89) (end 97.07 66.79) (width 0.2) (layer "F.Cu") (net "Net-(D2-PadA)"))
 (segment (start 130.82 74.72237) (end 128.09763 72) (width 0.2) (layer "F.Cu") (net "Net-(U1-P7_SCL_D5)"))
 (segment (start 128.09763 72) (end 126 72) (width 0.2) (layer "F.Cu") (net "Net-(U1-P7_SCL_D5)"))
 (segment (start 130.82 75.8) (end 130.82 74.72237) (width 0.2) (layer "F.Cu") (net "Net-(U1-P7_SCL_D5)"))
 (via (at 126 72) (size 0.6) (drill 0.3) (layers "F.Cu" "B.Cu") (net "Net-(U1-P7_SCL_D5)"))
 (segment (start 100.54 72.4) (end 98.54 70.4) (width 0.2) (layer "B.Cu") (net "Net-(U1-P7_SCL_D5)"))
 (segment (start 126 72) (end 101 72) (width 0.2) (layer "B.Cu") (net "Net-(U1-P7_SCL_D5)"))
 (segment (start 101 72) (end 100.6 72.4) (width 0.2) (layer "B.Cu") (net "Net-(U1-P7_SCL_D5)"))
 (segment (start 100.6 72.4) (end 100.54 72.4) (width 0.2) (layer "B.Cu") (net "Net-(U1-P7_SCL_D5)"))
 (segment (start 142.458 76.862) (end 80.948 76.862) (width 0.2) (layer "F.Cu") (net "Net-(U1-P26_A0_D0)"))
 (segment (start 80.948 76.862) (end 79.35 78.46) (width 0.2) (layer "F.Cu") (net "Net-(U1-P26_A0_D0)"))
 (segment (start 143.52 75.8) (end 142.458 76.862) (width 0.2) (layer "F.Cu") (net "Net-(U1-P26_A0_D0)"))
 (segment (start 139.71 77.07) (end 99.94 77.07) (width 0.2) (layer "B.Cu") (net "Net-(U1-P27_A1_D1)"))
 (segment (start 140.98 75.8) (end 139.71 77.07) (width 0.2) (layer "B.Cu") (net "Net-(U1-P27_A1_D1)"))
 (segment (start 99.94 77.07) (end 98.55 78.46) (width 0.2) (layer "B.Cu") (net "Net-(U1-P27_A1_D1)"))
 (segment (start 135.9 75.187786) (end 135.9 75.8) (width 0.2) (layer "F.Cu") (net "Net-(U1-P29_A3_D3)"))
 (segment (start 138.33 72.757786) (end 135.9 75.187786) (width 0.2) (layer "F.Cu") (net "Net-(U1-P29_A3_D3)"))
 (segment (start 138.33 57.55) (end 138.33 72.757786) (width 0.2) (layer "F.Cu") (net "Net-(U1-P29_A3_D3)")))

